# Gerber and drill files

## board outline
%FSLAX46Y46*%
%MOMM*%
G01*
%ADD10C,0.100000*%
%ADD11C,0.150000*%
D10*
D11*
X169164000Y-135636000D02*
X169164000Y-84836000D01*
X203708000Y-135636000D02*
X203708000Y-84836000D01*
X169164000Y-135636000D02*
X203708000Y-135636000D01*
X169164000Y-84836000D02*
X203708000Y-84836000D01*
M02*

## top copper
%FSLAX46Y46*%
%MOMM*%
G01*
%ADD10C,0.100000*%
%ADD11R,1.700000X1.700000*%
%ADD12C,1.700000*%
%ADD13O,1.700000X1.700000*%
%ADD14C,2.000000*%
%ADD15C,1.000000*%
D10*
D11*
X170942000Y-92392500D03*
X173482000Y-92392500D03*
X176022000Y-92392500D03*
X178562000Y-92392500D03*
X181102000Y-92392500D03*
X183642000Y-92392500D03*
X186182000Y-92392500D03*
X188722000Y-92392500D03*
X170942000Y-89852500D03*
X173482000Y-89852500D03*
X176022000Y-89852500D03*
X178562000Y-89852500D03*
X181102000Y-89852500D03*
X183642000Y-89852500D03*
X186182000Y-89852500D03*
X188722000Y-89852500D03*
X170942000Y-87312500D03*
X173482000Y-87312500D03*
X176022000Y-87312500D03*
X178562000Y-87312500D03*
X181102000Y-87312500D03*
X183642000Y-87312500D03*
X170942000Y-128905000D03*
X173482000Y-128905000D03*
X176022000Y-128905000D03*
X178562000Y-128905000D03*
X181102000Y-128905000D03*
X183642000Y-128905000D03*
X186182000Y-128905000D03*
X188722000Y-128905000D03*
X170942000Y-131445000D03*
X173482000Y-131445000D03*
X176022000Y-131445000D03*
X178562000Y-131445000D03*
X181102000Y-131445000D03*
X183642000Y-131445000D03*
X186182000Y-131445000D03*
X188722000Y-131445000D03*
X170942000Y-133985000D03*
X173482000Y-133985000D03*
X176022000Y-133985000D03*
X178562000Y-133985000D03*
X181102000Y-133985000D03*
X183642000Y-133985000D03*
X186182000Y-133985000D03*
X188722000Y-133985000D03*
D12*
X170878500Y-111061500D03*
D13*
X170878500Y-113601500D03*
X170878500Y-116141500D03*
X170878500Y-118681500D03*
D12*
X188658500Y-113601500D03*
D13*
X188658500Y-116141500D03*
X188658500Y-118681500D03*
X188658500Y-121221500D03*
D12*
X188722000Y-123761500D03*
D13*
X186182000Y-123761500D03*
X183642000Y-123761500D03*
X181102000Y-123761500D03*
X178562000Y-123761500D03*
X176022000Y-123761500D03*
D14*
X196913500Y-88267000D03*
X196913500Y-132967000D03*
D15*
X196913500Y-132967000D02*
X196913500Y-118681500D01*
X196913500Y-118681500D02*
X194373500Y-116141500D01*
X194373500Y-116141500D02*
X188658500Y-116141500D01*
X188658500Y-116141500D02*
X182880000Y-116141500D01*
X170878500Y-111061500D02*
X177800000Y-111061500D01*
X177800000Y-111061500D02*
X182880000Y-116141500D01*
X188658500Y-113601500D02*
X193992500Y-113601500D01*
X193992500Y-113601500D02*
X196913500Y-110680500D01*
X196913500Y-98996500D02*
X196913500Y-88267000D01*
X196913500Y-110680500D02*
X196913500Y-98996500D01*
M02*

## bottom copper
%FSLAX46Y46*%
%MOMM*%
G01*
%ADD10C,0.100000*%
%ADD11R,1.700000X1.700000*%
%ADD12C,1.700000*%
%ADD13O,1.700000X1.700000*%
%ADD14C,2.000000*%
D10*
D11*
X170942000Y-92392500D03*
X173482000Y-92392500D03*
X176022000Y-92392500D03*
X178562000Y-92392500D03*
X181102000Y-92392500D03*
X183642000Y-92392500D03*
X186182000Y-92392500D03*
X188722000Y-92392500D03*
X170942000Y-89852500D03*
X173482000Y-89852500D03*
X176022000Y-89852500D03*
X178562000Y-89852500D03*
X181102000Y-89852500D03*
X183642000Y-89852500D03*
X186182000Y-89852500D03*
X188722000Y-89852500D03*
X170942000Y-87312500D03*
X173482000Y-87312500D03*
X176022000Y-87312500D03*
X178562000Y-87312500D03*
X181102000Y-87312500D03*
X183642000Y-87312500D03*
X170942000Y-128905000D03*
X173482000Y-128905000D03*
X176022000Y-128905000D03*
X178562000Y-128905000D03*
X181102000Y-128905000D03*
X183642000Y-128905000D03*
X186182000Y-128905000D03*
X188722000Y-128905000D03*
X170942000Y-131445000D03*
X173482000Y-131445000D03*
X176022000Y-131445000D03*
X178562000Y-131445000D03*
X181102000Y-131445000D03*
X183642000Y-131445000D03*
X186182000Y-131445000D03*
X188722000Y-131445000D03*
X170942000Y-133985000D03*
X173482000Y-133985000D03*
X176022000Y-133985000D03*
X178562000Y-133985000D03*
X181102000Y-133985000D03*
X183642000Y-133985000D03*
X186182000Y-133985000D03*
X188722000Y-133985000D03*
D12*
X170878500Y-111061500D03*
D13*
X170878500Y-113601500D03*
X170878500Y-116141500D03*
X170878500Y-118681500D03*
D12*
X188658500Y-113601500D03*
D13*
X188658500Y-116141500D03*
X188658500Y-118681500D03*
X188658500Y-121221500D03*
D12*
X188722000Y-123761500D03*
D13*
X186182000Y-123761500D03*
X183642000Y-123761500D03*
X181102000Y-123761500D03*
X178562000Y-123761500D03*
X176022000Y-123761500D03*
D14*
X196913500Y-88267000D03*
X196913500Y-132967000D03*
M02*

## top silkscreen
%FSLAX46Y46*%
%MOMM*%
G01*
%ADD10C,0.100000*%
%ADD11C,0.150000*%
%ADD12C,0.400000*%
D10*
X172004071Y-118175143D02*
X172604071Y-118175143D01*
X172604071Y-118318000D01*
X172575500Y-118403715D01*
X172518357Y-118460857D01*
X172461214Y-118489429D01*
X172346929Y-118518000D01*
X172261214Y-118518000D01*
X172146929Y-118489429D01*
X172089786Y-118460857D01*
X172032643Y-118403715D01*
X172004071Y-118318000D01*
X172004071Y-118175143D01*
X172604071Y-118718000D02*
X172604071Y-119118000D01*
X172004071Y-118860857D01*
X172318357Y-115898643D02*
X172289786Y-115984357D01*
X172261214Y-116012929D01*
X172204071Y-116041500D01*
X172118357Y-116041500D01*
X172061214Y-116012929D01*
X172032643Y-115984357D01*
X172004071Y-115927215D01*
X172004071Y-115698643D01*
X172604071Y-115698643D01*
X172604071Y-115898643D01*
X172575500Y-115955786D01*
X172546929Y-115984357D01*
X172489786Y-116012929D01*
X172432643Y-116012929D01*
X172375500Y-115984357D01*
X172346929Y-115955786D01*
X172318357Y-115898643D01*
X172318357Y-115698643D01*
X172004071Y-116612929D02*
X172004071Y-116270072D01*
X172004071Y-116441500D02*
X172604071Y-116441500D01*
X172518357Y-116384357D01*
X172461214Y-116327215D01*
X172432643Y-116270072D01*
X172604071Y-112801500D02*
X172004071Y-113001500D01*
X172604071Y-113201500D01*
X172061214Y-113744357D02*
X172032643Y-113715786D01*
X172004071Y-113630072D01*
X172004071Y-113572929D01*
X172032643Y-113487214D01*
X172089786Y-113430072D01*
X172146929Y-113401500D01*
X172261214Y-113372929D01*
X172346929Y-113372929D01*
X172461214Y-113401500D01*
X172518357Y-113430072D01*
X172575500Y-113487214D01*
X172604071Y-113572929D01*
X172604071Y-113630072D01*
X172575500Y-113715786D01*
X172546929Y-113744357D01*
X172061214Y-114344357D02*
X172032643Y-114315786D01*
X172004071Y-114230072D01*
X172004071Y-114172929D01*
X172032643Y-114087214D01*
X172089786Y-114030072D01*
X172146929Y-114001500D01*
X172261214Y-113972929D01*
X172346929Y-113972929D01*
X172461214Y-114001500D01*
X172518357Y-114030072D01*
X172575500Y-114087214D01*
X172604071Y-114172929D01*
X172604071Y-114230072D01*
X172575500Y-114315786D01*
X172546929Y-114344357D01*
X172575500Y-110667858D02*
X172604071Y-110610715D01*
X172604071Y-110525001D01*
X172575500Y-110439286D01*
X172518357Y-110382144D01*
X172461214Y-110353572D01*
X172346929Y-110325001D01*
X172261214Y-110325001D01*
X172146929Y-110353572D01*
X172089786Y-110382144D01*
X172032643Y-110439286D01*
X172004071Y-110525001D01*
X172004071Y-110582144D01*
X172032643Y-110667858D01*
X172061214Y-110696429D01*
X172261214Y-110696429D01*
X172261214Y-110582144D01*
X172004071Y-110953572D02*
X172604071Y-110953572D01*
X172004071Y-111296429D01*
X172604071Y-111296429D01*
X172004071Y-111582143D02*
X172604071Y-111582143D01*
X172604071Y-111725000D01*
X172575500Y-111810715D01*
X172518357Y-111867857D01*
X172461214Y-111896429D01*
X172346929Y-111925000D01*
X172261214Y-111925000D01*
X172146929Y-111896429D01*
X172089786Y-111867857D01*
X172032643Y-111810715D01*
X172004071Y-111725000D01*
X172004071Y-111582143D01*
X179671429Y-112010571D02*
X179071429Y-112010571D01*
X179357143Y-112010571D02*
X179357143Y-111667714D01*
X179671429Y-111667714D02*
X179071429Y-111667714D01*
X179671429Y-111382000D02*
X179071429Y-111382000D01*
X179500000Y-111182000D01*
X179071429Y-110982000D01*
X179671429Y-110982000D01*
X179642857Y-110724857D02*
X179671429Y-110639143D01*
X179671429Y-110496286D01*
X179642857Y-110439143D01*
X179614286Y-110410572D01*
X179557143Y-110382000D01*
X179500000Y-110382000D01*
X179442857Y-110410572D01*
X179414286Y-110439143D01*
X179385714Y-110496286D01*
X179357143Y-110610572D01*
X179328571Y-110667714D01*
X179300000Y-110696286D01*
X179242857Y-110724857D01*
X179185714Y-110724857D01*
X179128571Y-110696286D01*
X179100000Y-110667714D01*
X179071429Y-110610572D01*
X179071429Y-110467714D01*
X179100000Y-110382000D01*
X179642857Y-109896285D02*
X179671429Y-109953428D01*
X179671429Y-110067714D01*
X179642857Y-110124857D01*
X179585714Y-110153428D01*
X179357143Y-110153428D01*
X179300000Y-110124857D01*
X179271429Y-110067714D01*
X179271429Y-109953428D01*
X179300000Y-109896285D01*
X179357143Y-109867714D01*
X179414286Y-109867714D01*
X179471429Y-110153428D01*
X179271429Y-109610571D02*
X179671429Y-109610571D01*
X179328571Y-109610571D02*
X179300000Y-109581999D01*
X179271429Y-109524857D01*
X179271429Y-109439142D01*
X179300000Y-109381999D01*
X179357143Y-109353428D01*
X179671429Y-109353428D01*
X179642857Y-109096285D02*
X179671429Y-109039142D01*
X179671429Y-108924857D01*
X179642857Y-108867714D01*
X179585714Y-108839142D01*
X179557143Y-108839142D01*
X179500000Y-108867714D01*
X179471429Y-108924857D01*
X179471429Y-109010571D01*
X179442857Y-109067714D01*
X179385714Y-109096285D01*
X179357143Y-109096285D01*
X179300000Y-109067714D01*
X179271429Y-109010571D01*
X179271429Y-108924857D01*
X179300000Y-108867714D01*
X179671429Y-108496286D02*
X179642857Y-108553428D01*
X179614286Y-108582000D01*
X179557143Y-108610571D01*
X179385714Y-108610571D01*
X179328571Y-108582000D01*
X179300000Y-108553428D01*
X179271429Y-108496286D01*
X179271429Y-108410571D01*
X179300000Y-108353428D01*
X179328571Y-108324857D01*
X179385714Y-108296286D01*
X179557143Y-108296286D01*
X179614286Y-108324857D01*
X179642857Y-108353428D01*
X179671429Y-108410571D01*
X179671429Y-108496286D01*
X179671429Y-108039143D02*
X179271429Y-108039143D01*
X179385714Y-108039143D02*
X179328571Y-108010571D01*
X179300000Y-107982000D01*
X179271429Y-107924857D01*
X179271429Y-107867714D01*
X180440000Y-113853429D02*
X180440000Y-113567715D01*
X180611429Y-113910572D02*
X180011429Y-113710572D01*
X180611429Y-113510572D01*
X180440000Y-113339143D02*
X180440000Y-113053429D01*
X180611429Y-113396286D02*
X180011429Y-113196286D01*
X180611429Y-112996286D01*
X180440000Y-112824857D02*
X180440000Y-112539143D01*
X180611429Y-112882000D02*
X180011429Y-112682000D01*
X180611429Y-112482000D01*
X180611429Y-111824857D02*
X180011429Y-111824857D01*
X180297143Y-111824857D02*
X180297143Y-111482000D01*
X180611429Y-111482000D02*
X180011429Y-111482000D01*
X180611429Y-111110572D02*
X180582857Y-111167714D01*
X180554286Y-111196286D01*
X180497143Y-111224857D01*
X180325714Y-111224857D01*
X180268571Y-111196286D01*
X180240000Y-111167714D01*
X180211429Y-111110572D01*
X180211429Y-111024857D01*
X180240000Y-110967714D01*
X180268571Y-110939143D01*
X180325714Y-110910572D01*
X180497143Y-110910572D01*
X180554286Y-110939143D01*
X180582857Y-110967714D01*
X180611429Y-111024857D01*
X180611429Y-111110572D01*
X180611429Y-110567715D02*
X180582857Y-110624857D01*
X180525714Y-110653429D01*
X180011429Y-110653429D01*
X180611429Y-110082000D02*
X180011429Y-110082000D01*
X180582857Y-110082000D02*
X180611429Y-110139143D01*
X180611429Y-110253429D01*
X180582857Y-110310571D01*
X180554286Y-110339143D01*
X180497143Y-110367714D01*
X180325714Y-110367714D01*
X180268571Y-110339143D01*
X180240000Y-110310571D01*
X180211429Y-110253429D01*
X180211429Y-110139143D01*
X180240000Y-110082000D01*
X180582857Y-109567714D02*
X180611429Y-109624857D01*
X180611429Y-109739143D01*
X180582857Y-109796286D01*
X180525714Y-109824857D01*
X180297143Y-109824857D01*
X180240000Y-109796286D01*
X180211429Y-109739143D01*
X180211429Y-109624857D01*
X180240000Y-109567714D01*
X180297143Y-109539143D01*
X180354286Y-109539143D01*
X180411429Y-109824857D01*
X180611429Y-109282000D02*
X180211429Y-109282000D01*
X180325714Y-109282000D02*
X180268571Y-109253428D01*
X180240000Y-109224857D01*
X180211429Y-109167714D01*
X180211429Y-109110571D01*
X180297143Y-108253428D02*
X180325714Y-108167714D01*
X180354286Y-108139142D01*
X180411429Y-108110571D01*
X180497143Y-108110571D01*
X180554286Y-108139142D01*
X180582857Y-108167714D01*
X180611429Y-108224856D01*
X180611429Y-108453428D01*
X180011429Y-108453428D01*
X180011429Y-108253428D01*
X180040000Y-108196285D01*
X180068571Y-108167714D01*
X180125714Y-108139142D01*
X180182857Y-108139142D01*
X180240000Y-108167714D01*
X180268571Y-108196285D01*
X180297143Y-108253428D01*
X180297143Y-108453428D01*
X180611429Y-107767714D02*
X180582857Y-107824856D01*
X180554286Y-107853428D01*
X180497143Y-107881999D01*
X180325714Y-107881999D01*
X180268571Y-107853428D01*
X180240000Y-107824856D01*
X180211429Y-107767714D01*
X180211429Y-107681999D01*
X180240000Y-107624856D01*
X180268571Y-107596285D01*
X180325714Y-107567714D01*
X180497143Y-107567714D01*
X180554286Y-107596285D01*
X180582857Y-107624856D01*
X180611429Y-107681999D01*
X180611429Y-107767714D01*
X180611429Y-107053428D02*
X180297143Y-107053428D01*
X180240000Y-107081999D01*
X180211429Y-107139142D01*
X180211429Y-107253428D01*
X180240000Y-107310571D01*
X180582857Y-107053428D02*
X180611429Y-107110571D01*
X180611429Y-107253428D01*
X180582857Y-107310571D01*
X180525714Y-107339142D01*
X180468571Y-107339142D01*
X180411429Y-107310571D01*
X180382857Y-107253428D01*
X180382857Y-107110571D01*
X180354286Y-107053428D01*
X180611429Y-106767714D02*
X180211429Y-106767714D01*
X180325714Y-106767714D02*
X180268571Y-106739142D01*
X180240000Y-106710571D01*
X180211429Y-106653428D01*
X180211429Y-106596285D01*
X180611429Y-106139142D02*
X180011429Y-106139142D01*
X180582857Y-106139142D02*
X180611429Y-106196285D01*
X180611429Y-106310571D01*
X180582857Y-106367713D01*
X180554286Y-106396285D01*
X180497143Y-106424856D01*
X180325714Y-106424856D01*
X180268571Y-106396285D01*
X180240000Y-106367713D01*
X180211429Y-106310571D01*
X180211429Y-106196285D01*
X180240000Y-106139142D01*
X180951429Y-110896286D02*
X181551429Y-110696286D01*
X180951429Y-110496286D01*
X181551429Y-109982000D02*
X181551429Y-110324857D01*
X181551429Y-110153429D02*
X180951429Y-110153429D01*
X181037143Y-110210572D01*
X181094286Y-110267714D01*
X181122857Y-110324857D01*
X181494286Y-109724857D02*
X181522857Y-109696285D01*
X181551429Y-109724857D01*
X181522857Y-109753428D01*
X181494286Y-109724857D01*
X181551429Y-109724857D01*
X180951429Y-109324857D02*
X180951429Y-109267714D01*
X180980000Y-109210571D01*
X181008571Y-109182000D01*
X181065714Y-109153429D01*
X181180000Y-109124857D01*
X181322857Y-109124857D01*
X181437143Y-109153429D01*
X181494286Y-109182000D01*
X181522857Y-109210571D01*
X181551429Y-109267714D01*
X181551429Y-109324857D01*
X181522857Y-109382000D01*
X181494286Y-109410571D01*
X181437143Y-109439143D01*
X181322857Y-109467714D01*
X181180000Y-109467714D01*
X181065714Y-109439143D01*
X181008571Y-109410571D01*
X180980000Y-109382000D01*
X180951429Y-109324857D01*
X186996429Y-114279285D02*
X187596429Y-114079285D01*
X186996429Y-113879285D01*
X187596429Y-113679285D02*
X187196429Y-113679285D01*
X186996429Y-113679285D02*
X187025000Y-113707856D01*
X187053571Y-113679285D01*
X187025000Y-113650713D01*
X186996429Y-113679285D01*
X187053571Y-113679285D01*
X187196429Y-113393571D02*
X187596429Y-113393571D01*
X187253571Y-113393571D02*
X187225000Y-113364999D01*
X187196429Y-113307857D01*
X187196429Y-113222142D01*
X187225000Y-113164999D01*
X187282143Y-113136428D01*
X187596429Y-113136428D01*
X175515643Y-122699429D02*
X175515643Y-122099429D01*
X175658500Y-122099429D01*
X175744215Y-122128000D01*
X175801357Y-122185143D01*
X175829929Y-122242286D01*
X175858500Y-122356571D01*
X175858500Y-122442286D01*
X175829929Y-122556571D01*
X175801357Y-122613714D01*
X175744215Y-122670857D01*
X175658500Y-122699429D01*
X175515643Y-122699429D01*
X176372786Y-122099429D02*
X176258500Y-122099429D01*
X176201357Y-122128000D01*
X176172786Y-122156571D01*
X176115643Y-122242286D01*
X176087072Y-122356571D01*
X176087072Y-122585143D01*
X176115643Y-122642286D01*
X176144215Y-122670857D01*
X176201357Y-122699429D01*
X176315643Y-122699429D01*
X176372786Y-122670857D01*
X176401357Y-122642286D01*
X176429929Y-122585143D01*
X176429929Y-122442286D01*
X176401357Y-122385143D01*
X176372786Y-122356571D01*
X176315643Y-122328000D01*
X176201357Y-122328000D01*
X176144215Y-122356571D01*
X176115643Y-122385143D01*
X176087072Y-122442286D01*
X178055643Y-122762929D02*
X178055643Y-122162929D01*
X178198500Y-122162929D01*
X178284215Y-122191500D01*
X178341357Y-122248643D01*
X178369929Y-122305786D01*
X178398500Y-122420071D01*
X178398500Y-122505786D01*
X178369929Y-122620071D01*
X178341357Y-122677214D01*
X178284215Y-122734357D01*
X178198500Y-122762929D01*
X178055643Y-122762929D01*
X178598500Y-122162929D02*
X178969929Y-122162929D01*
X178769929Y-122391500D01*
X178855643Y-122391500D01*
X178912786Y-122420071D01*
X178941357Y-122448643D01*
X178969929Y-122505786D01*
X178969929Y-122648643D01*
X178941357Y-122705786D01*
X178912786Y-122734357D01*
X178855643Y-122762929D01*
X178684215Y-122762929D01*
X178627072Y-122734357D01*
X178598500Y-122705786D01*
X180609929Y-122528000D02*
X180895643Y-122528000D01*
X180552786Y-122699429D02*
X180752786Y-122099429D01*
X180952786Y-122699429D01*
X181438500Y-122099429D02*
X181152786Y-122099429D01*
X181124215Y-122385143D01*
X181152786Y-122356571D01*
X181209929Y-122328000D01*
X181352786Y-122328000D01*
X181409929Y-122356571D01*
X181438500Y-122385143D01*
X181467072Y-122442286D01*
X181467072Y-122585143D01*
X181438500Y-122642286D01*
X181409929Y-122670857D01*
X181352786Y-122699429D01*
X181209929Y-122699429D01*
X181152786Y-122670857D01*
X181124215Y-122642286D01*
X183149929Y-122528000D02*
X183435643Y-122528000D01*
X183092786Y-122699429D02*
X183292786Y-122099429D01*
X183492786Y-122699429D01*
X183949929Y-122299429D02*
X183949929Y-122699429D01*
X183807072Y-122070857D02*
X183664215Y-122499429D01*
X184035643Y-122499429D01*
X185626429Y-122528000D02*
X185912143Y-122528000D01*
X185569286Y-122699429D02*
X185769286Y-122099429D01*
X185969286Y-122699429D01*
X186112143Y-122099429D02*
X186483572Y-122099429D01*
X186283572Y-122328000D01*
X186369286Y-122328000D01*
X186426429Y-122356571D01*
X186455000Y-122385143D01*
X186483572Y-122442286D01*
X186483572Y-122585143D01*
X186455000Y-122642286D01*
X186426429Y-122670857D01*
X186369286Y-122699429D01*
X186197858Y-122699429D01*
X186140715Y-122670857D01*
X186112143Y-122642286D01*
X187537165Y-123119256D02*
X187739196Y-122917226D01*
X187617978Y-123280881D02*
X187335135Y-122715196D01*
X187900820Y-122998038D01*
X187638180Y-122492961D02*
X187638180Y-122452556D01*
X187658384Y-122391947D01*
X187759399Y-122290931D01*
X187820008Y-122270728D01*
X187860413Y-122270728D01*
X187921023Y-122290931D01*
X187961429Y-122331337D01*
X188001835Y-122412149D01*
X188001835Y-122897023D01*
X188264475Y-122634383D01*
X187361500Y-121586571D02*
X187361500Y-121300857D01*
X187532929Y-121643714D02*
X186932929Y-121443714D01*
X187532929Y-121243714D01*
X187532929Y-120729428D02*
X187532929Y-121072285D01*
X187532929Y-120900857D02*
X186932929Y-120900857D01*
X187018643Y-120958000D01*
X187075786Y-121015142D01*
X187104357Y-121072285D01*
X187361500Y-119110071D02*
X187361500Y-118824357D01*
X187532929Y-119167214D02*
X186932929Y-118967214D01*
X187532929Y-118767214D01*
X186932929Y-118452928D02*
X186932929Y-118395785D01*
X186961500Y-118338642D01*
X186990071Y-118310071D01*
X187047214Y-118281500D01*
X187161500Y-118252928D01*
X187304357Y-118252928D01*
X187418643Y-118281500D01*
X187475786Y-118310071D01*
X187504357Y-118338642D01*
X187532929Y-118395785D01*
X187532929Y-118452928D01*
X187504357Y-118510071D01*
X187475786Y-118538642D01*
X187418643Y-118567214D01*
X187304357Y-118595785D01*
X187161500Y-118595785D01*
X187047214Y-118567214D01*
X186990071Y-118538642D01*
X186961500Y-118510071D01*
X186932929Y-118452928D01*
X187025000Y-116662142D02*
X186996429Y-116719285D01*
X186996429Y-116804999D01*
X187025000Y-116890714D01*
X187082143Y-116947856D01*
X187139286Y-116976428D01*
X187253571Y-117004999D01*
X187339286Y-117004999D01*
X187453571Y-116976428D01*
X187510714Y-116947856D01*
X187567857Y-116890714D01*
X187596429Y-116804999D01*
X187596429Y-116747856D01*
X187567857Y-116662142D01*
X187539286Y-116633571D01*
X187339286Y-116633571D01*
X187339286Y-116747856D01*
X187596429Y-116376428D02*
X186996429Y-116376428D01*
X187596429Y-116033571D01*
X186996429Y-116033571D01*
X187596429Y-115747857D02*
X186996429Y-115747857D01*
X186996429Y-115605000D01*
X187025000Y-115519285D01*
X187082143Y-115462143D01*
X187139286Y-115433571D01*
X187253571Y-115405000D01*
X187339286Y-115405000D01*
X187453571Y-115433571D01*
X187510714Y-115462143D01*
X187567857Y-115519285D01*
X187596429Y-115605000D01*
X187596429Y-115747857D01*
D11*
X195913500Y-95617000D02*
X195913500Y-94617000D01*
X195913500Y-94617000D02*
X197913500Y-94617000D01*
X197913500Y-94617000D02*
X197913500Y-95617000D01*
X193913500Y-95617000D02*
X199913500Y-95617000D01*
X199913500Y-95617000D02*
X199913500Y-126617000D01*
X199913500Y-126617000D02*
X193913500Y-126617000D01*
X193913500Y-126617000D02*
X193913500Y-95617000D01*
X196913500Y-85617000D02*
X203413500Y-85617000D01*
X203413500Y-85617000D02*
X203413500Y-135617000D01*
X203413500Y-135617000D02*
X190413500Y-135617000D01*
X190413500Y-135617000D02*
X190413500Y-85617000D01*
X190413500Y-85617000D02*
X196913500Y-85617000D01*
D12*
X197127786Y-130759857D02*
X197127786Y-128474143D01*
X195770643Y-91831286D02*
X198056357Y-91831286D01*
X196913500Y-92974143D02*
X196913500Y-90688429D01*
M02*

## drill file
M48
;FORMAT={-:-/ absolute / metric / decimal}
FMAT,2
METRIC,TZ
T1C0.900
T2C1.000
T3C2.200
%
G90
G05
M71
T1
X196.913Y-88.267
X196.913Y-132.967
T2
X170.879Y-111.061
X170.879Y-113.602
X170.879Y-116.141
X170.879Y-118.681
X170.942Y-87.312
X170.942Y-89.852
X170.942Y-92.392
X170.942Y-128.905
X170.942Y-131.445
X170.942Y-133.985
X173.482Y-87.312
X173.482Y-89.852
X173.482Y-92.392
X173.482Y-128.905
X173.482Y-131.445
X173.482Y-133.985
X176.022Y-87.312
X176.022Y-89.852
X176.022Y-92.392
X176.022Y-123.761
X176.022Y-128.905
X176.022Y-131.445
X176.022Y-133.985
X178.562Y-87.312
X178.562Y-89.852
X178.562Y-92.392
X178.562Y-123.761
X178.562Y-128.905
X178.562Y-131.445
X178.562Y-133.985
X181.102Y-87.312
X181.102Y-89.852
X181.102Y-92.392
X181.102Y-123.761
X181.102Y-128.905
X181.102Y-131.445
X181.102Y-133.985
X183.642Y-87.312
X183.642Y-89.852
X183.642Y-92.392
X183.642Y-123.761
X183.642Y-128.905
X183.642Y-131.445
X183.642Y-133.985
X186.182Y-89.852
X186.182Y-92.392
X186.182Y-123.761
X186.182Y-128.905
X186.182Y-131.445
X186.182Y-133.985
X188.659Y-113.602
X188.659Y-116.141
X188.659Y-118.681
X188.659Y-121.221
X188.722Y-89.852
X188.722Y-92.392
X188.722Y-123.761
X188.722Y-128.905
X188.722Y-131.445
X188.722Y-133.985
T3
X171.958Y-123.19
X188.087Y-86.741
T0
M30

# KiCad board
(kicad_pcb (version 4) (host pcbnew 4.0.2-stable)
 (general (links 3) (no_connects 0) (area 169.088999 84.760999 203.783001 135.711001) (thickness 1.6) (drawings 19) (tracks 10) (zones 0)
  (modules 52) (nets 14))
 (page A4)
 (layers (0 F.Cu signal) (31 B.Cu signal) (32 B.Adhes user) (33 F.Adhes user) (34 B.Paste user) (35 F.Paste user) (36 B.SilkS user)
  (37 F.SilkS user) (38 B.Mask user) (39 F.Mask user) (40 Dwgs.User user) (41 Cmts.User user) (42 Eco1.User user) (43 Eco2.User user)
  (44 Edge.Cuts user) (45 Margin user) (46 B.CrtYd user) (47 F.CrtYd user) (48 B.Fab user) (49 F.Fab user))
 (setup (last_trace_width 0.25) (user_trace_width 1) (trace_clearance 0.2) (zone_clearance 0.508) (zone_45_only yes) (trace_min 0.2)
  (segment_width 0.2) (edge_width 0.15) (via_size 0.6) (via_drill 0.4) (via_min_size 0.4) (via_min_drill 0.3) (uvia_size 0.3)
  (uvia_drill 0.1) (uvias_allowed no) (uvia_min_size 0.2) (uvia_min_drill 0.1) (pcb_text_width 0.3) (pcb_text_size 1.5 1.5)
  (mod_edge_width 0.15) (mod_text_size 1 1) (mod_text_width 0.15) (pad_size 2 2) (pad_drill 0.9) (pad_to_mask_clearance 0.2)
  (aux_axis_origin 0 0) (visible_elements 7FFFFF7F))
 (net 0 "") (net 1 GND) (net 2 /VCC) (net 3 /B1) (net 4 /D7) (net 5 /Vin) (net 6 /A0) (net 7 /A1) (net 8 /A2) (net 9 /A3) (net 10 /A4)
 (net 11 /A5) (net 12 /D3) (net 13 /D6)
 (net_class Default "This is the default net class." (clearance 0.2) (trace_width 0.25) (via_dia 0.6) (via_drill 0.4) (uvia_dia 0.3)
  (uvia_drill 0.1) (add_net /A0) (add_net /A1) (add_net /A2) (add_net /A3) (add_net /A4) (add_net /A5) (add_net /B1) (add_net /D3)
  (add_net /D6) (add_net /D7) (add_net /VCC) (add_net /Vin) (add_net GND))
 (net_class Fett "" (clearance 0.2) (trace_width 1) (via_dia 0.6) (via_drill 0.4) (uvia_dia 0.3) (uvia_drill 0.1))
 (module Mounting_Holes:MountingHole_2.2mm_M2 (layer F.Cu) (at 188.087 86.741)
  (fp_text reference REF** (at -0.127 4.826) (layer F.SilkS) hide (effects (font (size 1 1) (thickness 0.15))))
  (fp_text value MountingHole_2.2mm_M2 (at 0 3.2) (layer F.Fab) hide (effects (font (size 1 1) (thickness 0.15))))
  (pad 1 np_thru_hole circle (at 0 0) (size 2.2 2.2) (drill 2.2) (layers *.Cu *.Mask)))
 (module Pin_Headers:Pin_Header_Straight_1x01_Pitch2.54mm (layer F.Cu) (at 170.942 92.3925)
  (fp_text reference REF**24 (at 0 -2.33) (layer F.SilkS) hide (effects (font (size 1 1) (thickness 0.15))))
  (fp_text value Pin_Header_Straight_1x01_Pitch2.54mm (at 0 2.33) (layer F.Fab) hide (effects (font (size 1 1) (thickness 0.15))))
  (pad 1 thru_hole rect (at 0 0) (size 1.7 1.7) (drill 1) (layers *.Cu *.Mask)))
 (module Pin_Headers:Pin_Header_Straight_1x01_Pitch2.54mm (layer F.Cu) (at 173.482 92.3925)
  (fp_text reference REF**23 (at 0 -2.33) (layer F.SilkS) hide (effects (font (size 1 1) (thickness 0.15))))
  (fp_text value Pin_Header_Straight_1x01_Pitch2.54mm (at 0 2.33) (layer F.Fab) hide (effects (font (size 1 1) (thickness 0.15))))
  (pad 1 thru_hole rect (at 0 0) (size 1.7 1.7) (drill 1) (layers *.Cu *.Mask)))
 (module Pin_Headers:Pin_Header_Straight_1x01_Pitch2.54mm (layer F.Cu) (at 176.022 92.3925)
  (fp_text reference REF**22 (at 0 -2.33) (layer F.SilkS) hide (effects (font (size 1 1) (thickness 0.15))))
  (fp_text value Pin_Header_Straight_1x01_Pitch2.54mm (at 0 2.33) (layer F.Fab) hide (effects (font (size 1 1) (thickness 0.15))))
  (pad 1 thru_hole rect (at 0 0) (size 1.7 1.7) (drill 1) (layers *.Cu *.Mask)))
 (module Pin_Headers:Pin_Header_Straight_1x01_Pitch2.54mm (layer F.Cu) (at 178.562 92.3925)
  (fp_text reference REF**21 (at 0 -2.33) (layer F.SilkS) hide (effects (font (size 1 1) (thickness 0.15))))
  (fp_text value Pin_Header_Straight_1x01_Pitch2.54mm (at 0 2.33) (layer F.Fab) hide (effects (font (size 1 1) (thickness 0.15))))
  (pad 1 thru_hole rect (at 0 0) (size 1.7 1.7) (drill 1) (layers *.Cu *.Mask)))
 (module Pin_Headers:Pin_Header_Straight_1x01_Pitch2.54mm (layer F.Cu) (at 181.102 92.3925)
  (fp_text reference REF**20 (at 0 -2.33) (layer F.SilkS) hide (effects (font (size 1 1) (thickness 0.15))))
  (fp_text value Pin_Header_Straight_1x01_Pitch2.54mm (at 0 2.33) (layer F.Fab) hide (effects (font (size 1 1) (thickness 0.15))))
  (pad 1 thru_hole rect (at 0 0) (size 1.7 1.7) (drill 1) (layers *.Cu *.Mask)))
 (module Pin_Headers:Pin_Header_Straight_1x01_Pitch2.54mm (layer F.Cu) (at 183.642 92.3925)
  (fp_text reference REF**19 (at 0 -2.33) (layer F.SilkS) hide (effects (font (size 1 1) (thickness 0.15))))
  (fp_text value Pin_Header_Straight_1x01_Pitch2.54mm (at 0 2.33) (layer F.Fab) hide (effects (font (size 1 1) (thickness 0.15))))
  (pad 1 thru_hole rect (at 0 0) (size 1.7 1.7) (drill 1) (layers *.Cu *.Mask)))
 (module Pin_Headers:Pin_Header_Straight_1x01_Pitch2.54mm (layer F.Cu) (at 186.182 92.3925)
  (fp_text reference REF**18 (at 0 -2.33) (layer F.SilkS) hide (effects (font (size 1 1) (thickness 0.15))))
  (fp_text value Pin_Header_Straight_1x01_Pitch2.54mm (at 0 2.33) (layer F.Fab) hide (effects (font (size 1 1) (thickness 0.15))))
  (pad 1 thru_hole rect (at 0 0) (size 1.7 1.7) (drill 1) (layers *.Cu *.Mask)))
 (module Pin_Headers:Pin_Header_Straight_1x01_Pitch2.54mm (layer F.Cu) (at 188.722 92.3925)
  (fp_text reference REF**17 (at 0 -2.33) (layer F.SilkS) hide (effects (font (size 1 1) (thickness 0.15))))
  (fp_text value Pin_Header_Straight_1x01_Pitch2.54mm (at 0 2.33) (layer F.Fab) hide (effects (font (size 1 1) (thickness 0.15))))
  (pad 1 thru_hole rect (at 0 0) (size 1.7 1.7) (drill 1) (layers *.Cu *.Mask)))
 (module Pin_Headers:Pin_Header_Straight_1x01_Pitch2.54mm (layer F.Cu) (at 170.942 89.8525)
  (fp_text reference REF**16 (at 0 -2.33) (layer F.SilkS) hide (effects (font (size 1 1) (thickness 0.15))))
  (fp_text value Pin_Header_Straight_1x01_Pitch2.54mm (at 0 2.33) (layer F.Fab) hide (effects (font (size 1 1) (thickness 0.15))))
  (pad 1 thru_hole rect (at 0 0) (size 1.7 1.7) (drill 1) (layers *.Cu *.Mask)))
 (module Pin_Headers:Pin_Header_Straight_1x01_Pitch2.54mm (layer F.Cu) (at 173.482 89.8525)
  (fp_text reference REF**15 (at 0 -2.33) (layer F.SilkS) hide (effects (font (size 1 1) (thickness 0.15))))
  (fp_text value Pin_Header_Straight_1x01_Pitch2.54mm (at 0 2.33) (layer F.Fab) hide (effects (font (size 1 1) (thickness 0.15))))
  (pad 1 thru_hole rect (at 0 0) (size 1.7 1.7) (drill 1) (layers *.Cu *.Mask)))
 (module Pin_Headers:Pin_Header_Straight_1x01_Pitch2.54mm (layer F.Cu) (at 176.022 89.8525)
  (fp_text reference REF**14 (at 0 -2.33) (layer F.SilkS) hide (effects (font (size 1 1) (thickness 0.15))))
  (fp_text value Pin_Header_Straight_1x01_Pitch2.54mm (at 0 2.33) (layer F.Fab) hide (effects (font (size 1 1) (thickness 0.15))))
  (pad 1 thru_hole rect (at 0 0) (size 1.7 1.7) (drill 1) (layers *.Cu *.Mask)))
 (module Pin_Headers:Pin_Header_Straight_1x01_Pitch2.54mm (layer F.Cu) (at 178.562 89.8525)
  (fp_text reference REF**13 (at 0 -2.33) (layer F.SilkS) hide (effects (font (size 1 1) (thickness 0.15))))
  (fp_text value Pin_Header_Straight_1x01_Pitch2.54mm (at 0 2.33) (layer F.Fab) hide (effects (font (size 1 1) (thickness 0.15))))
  (pad 1 thru_hole rect (at 0 0) (size 1.7 1.7) (drill 1) (layers *.Cu *.Mask)))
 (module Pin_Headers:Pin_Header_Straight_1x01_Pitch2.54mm (layer F.Cu) (at 181.102 89.8525)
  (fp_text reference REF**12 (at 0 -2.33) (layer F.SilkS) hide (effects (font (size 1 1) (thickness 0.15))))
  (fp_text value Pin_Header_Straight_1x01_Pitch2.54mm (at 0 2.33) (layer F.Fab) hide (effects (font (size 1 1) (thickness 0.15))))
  (pad 1 thru_hole rect (at 0 0) (size 1.7 1.7) (drill 1) (layers *.Cu *.Mask)))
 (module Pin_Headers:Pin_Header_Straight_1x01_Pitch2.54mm (layer F.Cu) (at 183.642 89.8525)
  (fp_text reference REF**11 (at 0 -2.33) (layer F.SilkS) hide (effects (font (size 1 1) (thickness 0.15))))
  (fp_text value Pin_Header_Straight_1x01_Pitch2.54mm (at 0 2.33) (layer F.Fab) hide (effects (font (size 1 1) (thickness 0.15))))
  (pad 1 thru_hole rect (at 0 0) (size 1.7 1.7) (drill 1) (layers *.Cu *.Mask)))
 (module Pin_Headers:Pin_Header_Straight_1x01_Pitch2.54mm (layer F.Cu) (at 186.182 89.8525)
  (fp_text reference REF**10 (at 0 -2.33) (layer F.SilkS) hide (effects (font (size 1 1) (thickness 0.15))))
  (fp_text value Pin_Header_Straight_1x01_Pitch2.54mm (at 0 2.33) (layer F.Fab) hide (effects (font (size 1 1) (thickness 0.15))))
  (pad 1 thru_hole rect (at 0 0) (size 1.7 1.7) (drill 1) (layers *.Cu *.Mask)))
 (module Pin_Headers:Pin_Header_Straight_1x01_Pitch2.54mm (layer F.Cu) (at 188.722 89.8525)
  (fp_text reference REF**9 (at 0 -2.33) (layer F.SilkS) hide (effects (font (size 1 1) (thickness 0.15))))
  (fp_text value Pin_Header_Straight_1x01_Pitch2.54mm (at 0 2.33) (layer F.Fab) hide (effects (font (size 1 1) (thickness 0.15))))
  (pad 1 thru_hole rect (at 0 0) (size 1.7 1.7) (drill 1) (layers *.Cu *.Mask)))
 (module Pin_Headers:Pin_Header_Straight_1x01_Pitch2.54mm (layer F.Cu) (at 170.942 87.3125)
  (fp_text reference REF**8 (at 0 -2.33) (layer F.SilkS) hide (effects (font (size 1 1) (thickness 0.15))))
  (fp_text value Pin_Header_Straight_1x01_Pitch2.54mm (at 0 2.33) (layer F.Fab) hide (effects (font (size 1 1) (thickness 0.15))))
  (pad 1 thru_hole rect (at 0 0) (size 1.7 1.7) (drill 1) (layers *.Cu *.Mask)))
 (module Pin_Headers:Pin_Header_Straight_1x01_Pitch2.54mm (layer F.Cu) (at 173.482 87.3125)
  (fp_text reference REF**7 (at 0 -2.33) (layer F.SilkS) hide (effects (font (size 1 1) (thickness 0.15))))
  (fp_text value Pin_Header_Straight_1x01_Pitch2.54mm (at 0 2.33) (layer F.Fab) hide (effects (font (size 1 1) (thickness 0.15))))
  (pad 1 thru_hole rect (at 0 0) (size 1.7 1.7) (drill 1) (layers *.Cu *.Mask)))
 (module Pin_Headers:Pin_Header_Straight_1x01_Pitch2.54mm (layer F.Cu) (at 176.022 87.3125)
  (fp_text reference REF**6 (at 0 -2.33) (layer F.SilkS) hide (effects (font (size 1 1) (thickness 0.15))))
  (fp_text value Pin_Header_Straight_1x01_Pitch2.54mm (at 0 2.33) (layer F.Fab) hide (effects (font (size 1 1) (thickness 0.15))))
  (pad 1 thru_hole rect (at 0 0) (size 1.7 1.7) (drill 1) (layers *.Cu *.Mask)))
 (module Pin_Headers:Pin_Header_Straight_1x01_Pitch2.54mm (layer F.Cu) (at 178.562 87.3125)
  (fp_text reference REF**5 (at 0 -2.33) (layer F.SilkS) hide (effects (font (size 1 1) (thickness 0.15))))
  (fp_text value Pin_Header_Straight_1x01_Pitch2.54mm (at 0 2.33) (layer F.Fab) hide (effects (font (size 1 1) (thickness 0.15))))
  (pad 1 thru_hole rect (at 0 0) (size 1.7 1.7) (drill 1) (layers *.Cu *.Mask)))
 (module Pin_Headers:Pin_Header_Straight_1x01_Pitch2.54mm (layer F.Cu) (at 181.102 87.3125)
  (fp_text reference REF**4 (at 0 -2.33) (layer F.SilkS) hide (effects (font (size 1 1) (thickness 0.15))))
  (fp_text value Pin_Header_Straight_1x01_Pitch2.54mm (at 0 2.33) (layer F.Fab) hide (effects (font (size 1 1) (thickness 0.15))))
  (pad 1 thru_hole rect (at 0 0) (size 1.7 1.7) (drill 1) (layers *.Cu *.Mask)))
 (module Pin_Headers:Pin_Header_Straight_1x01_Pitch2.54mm (layer F.Cu) (at 183.642 87.3125)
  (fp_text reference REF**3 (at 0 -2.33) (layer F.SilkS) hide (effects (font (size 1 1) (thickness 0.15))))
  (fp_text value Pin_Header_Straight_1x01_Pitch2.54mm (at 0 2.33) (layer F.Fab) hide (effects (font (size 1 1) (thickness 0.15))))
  (pad 1 thru_hole rect (at 0 0) (size 1.7 1.7) (drill 1) (layers *.Cu *.Mask)))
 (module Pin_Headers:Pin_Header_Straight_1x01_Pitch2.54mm (layer F.Cu) (at 170.942 128.905)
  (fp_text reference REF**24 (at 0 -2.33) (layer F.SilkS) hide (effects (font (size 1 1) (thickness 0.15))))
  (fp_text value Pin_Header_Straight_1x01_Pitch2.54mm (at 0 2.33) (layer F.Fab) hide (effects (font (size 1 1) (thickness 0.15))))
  (pad 1 thru_hole rect (at 0 0) (size 1.7 1.7) (drill 1) (layers *.Cu *.Mask)))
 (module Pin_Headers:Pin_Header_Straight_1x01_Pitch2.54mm (layer F.Cu) (at 173.482 128.905)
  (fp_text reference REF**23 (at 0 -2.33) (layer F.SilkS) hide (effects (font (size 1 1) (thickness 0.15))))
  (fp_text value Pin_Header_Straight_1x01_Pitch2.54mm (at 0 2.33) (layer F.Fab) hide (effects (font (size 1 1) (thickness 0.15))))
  (pad 1 thru_hole rect (at 0 0) (size 1.7 1.7) (drill 1) (layers *.Cu *.Mask)))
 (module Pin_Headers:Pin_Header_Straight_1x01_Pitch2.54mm (layer F.Cu) (at 176.022 128.905)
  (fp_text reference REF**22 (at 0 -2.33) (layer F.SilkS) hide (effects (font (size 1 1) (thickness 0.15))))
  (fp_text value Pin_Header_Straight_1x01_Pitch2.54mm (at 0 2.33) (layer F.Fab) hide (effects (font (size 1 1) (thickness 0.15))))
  (pad 1 thru_hole rect (at 0 0) (size 1.7 1.7) (drill 1) (layers *.Cu *.Mask)))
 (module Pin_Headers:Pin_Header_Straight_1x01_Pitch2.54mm (layer F.Cu) (at 178.562 128.905)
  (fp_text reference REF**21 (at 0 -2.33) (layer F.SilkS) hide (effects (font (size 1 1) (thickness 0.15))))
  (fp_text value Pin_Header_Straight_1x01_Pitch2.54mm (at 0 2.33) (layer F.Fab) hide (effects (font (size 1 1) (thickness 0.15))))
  (pad 1 thru_hole rect (at 0 0) (size 1.7 1.7) (drill 1) (layers *.Cu *.Mask)))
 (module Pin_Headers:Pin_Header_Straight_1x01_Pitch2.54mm (layer F.Cu) (at 181.102 128.905)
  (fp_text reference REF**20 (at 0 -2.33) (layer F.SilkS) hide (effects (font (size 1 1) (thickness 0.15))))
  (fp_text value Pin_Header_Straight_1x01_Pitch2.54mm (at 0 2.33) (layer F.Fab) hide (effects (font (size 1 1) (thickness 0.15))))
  (pad 1 thru_hole rect (at 0 0) (size 1.7 1.7) (drill 1) (layers *.Cu *.Mask)))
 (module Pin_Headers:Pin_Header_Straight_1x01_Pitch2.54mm (layer F.Cu) (at 183.642 128.905)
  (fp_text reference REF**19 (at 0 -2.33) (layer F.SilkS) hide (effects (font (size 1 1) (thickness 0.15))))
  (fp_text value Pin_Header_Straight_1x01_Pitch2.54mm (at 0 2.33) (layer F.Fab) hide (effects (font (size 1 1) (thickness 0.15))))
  (pad 1 thru_hole rect (at 0 0) (size 1.7 1.7) (drill 1) (layers *.Cu *.Mask)))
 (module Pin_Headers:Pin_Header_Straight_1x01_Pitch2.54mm (layer F.Cu) (at 186.182 128.905)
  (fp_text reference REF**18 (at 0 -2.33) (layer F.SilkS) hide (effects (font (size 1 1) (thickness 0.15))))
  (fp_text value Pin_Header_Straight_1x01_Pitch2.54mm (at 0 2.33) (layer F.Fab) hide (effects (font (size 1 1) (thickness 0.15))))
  (pad 1 thru_hole rect (at 0 0) (size 1.7 1.7) (drill 1) (layers *.Cu *.Mask)))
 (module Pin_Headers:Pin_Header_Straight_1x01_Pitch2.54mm (layer F.Cu) (at 188.722 128.905)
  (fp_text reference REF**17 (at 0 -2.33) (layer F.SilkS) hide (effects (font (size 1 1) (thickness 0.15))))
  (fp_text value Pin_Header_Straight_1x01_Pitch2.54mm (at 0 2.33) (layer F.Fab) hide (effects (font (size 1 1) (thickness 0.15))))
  (pad 1 thru_hole rect (at 0 0) (size 1.7 1.7) (drill 1) (layers *.Cu *.Mask)))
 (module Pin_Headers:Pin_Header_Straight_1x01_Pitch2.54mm (layer F.Cu) (at 170.942 131.445)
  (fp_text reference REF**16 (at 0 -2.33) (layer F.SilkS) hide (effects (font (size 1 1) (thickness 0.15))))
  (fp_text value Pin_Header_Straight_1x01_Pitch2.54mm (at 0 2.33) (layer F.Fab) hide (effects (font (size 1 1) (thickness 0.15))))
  (pad 1 thru_hole rect (at 0 0) (size 1.7 1.7) (drill 1) (layers *.Cu *.Mask)))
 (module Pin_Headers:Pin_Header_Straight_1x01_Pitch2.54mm (layer F.Cu) (at 173.482 131.445)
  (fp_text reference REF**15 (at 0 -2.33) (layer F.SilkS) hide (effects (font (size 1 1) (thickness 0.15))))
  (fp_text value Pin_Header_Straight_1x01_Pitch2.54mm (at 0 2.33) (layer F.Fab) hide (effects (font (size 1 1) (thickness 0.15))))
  (pad 1 thru_hole rect (at 0 0) (size 1.7 1.7) (drill 1) (layers *.Cu *.Mask)))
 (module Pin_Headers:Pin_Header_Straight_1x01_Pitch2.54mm (layer F.Cu) (at 176.022 131.445)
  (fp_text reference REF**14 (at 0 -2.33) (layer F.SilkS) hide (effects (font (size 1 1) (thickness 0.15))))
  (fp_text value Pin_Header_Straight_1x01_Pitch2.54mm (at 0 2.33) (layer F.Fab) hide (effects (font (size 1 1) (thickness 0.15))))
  (pad 1 thru_hole rect (at 0 0) (size 1.7 1.7) (drill 1) (layers *.Cu *.Mask)))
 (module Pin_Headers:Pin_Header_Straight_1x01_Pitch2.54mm (layer F.Cu) (at 178.562 131.445)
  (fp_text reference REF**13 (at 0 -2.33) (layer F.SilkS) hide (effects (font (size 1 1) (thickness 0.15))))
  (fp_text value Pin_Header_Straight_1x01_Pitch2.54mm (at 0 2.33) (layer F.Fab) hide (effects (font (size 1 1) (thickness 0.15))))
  (pad 1 thru_hole rect (at 0 0) (size 1.7 1.7) (drill 1) (layers *.Cu *.Mask)))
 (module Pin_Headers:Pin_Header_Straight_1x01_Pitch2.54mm (layer F.Cu) (at 181.102 131.445)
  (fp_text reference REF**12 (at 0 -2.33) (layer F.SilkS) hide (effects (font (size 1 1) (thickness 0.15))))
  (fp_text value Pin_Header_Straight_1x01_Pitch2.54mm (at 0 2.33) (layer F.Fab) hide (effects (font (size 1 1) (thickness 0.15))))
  (pad 1 thru_hole rect (at 0 0) (size 1.7 1.7) (drill 1) (layers *.Cu *.Mask)))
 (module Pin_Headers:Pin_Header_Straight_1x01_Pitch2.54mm (layer F.Cu) (at 183.642 131.445)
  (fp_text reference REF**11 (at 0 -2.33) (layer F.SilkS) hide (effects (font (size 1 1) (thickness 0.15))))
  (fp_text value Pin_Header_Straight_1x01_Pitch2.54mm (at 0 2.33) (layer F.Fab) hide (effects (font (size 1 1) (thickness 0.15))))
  (pad 1 thru_hole rect (at 0 0) (size 1.7 1.7) (drill 1) (layers *.Cu *.Mask)))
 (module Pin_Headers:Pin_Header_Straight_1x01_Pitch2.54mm (layer F.Cu) (at 186.182 131.445)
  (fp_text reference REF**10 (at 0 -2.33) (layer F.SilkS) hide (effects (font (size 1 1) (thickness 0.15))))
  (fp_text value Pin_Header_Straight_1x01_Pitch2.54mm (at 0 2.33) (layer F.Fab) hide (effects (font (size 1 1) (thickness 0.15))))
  (pad 1 thru_hole rect (at 0 0) (size 1.7 1.7) (drill 1) (layers *.Cu *.Mask)))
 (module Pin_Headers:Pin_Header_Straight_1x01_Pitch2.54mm (layer F.Cu) (at 188.722 131.445)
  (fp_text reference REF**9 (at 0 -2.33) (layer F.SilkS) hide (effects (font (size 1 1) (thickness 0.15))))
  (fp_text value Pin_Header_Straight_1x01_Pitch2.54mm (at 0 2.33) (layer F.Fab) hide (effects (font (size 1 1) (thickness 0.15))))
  (pad 1 thru_hole rect (at 0 0) (size 1.7 1.7) (drill 1) (layers *.Cu *.Mask)))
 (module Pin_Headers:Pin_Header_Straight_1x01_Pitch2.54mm (layer F.Cu) (at 170.942 133.985)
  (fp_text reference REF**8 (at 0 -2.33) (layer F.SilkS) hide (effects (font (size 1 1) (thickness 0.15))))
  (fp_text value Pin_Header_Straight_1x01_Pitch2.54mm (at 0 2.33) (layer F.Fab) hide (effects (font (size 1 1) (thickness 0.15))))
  (pad 1 thru_hole rect (at 0 0) (size 1.7 1.7) (drill 1) (layers *.Cu *.Mask)))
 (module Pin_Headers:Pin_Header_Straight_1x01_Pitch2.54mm (layer F.Cu) (at 173.482 133.985)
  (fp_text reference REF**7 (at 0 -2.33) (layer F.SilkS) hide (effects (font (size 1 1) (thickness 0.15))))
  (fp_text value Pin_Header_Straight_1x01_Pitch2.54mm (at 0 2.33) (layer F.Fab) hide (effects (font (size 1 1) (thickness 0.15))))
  (pad 1 thru_hole rect (at 0 0) (size 1.7 1.7) (drill 1) (layers *.Cu *.Mask)))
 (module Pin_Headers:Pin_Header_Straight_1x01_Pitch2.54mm (layer F.Cu) (at 176.022 133.985)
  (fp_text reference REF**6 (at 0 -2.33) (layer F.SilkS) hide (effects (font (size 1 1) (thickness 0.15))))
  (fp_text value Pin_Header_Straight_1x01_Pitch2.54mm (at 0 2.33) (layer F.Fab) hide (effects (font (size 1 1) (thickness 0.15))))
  (pad 1 thru_hole rect (at 0 0) (size 1.7 1.7) (drill 1) (layers *.Cu *.Mask)))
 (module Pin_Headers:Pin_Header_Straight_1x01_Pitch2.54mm (layer F.Cu) (at 178.562 133.985)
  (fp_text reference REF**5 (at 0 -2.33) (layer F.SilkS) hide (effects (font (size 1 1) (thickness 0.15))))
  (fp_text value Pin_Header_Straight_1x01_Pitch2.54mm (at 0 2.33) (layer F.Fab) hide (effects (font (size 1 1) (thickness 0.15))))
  (pad 1 thru_hole rect (at 0 0) (size 1.7 1.7) (drill 1) (layers *.Cu *.Mask)))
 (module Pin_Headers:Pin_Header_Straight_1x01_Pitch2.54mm (layer F.Cu) (at 181.102 133.985)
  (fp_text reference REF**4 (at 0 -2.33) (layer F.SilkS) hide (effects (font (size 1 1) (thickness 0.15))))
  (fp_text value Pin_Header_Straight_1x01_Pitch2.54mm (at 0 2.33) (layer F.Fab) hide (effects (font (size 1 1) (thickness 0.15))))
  (pad 1 thru_hole rect (at 0 0) (size 1.7 1.7) (drill 1) (layers *.Cu *.Mask)))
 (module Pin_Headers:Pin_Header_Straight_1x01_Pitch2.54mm (layer F.Cu) (at 183.642 133.985)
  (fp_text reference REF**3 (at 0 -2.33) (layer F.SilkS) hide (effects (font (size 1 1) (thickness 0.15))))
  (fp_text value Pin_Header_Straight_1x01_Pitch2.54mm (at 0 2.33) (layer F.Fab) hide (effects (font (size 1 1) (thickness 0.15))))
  (pad 1 thru_hole rect (at 0 0) (size 1.7 1.7) (drill 1) (layers *.Cu *.Mask)))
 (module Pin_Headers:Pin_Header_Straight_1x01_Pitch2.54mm (layer F.Cu) (at 186.182 133.985)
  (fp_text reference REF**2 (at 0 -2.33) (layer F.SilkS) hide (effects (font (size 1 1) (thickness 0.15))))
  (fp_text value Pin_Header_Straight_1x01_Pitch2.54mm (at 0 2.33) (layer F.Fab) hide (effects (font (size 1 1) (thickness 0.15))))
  (pad 1 thru_hole rect (at 0 0) (size 1.7 1.7) (drill 1) (layers *.Cu *.Mask)))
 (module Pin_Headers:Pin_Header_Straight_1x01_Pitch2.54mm (layer F.Cu) (at 188.722 133.985)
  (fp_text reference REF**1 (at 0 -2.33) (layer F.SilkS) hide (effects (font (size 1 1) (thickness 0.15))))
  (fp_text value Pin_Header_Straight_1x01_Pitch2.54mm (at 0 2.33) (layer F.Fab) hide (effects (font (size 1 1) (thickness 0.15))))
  (pad 1 thru_hole rect (at 0 0) (size 1.7 1.7) (drill 1) (layers *.Cu *.Mask)))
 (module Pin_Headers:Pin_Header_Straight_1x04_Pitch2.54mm (layer F.Cu) (at 170.8785 111.0615)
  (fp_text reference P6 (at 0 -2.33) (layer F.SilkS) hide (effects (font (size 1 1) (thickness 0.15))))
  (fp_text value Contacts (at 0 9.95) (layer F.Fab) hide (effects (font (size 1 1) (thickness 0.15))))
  (pad 1 thru_hole circle (at 0 0) (size 1.7 1.7) (drill 1) (layers *.Cu *.Mask) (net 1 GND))
  (pad 2 thru_hole oval (at 0 2.54) (size 1.7 1.7) (drill 1) (layers *.Cu *.Mask) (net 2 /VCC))
  (pad 3 thru_hole oval (at 0 5.08) (size 1.7 1.7) (drill 1) (layers *.Cu *.Mask) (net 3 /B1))
  (pad 4 thru_hole oval (at 0 7.62) (size 1.7 1.7) (drill 1) (layers *.Cu *.Mask) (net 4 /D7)))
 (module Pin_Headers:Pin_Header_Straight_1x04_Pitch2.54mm (layer F.Cu) (at 188.6585 113.6015)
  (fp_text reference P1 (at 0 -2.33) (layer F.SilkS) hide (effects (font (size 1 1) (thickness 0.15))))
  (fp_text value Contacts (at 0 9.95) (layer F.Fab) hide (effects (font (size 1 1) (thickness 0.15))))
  (pad 1 thru_hole circle (at 0 0) (size 1.7 1.7) (drill 1) (layers *.Cu *.Mask) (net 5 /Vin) (zone_connect 2))
  (pad 2 thru_hole oval (at 0 2.54) (size 1.7 1.7) (drill 1) (layers *.Cu *.Mask) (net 1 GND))
  (pad 3 thru_hole oval (at 0 5.08) (size 1.7 1.7) (drill 1) (layers *.Cu *.Mask) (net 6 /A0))
  (pad 4 thru_hole oval (at 0 7.62) (size 1.7 1.7) (drill 1) (layers *.Cu *.Mask) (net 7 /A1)))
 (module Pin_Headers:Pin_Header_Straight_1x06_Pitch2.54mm (layer F.Cu) (at 188.722 123.7615 270)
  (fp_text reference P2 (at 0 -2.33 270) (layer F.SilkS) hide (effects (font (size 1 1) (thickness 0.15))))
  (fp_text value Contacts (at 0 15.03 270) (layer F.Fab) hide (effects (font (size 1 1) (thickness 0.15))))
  (pad 1 thru_hole circle (at 0 0 270) (size 1.7 1.7) (drill 1) (layers *.Cu *.Mask) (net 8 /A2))
  (pad 2 thru_hole oval (at 0 2.54 270) (size 1.7 1.7) (drill 1) (layers *.Cu *.Mask) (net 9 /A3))
  (pad 3 thru_hole oval (at 0 5.08 270) (size 1.7 1.7) (drill 1) (layers *.Cu *.Mask) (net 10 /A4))
  (pad 4 thru_hole oval (at 0 7.62 270) (size 1.7 1.7) (drill 1) (layers *.Cu *.Mask) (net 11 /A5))
  (pad 5 thru_hole oval (at 0 10.16 270) (size 1.7 1.7) (drill 1) (layers *.Cu *.Mask) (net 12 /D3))
  (pad 6 thru_hole oval (at 0 12.7 270) (size 1.7 1.7) (drill 1) (layers *.Cu *.Mask) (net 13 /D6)))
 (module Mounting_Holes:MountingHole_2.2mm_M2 (layer F.Cu) (at 171.958 123.19)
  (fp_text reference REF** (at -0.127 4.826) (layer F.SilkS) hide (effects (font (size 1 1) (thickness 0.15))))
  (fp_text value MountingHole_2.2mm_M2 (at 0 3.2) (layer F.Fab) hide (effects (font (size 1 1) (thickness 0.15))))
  (pad 1 np_thru_hole circle (at 0 0) (size 2.2 2.2) (drill 2.2) (layers *.Cu *.Mask)))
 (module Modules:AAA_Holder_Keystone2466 (layer F.Cu) (at 196.9135 110.617)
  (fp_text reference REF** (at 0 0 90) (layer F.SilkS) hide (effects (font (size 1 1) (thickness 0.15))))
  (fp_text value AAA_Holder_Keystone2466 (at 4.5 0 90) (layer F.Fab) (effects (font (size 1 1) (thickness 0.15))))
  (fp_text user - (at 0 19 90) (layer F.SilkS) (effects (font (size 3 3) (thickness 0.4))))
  (fp_line (start -1 -15) (end -1 -16) (layer F.SilkS) (width 0.15))
  (fp_line (start -1 -16) (end 1 -16) (layer F.SilkS) (width 0.15))
  (fp_line (start 1 -16) (end 1 -15) (layer F.SilkS) (width 0.15))
  (fp_line (start -3 -15) (end 3 -15) (layer F.SilkS) (width 0.15))
  (fp_line (start 3 -15) (end 3 16) (layer F.SilkS) (width 0.15))
  (fp_line (start 3 16) (end -3 16) (layer F.SilkS) (width 0.15))
  (fp_line (start -3 16) (end -3 -15) (layer F.SilkS) (width 0.15))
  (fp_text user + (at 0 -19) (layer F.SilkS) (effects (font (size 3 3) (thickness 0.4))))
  (fp_line (start 0 -25) (end 6.5 -25) (layer F.SilkS) (width 0.15))
  (fp_line (start 6.5 -25) (end 6.5 25) (layer F.SilkS) (width 0.15))
  (fp_line (start 6.5 25) (end -6.5 25) (layer F.SilkS) (width 0.15))
  (fp_line (start -6.5 25) (end -6.5 -25) (layer F.SilkS) (width 0.15))
  (fp_line (start -6.5 -25) (end 0 -25) (layer F.SilkS) (width 0.15))
  (pad 1 thru_hole circle (at 0 -22.35) (size 2 2) (drill 0.9) (layers *.Cu *.Mask F.SilkS) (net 5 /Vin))
  (pad 2 thru_hole circle (at 0 22.35) (size 2 2) (drill 0.9) (layers *.Cu *.Mask F.SilkS) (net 1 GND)))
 (gr_line (start 169.164 135.636) (end 169.164 84.836) (angle 90) (layer Edge.Cuts) (width 0.15))
 (gr_line (start 203.708 135.636) (end 203.708 84.836) (angle 90) (layer Edge.Cuts) (width 0.15))
 (gr_line (start 169.164 135.636) (end 203.708 135.636) (angle 90) (layer Edge.Cuts) (width 0.15))
 (gr_line (start 169.164 84.836) (end 203.708 84.836) (angle 90) (layer Edge.Cuts) (width 0.15))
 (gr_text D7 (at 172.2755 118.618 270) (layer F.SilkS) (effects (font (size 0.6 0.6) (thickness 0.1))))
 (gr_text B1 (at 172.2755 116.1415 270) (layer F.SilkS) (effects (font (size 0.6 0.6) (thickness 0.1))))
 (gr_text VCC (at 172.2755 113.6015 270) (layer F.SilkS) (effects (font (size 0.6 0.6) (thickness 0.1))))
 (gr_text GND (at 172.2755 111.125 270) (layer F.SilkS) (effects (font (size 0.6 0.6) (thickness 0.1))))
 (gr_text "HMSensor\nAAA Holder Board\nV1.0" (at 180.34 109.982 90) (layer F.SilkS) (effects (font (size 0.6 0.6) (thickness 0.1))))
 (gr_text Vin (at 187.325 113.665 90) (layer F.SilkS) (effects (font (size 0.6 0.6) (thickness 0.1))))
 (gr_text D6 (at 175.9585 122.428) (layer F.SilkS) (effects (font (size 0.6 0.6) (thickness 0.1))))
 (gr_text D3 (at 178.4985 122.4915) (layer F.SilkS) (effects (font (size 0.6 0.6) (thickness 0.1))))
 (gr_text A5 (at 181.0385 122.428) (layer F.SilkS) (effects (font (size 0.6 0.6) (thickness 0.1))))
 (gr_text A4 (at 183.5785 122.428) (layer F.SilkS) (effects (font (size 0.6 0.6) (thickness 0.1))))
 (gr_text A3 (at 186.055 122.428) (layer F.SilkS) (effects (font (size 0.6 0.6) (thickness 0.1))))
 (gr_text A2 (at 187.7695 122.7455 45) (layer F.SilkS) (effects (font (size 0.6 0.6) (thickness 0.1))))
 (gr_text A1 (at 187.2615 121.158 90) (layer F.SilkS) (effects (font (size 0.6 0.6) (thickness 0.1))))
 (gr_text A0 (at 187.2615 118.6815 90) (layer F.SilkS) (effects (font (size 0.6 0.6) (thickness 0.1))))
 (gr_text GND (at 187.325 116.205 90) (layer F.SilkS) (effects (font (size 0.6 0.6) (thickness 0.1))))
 (segment (start 196.9135 132.967) (end 196.9135 118.6815) (width 1) (layer F.Cu) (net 1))
 (segment (start 196.9135 118.6815) (end 194.3735 116.1415) (width 1) (layer F.Cu) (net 1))
 (segment (start 194.3735 116.1415) (end 188.6585 116.1415) (width 1) (layer F.Cu) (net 1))
 (segment (start 188.6585 116.1415) (end 182.88 116.1415) (width 1) (layer F.Cu) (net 1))
 (segment (start 170.8785 111.0615) (end 177.8 111.0615) (width 1) (layer F.Cu) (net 1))
 (segment (start 177.8 111.0615) (end 182.88 116.1415) (width 1) (layer F.Cu) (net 1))
 (segment (start 188.6585 113.6015) (end 193.9925 113.6015) (width 1) (layer F.Cu) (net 5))
 (segment (start 193.9925 113.6015) (end 196.9135 110.6805) (width 1) (layer F.Cu) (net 5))
 (segment (start 196.9135 98.9965) (end 196.9135 88.267) (width 1) (layer F.Cu) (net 5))
 (segment (start 196.9135 110.6805) (end 196.9135 98.9965) (width 1) (layer F.Cu) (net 5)))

